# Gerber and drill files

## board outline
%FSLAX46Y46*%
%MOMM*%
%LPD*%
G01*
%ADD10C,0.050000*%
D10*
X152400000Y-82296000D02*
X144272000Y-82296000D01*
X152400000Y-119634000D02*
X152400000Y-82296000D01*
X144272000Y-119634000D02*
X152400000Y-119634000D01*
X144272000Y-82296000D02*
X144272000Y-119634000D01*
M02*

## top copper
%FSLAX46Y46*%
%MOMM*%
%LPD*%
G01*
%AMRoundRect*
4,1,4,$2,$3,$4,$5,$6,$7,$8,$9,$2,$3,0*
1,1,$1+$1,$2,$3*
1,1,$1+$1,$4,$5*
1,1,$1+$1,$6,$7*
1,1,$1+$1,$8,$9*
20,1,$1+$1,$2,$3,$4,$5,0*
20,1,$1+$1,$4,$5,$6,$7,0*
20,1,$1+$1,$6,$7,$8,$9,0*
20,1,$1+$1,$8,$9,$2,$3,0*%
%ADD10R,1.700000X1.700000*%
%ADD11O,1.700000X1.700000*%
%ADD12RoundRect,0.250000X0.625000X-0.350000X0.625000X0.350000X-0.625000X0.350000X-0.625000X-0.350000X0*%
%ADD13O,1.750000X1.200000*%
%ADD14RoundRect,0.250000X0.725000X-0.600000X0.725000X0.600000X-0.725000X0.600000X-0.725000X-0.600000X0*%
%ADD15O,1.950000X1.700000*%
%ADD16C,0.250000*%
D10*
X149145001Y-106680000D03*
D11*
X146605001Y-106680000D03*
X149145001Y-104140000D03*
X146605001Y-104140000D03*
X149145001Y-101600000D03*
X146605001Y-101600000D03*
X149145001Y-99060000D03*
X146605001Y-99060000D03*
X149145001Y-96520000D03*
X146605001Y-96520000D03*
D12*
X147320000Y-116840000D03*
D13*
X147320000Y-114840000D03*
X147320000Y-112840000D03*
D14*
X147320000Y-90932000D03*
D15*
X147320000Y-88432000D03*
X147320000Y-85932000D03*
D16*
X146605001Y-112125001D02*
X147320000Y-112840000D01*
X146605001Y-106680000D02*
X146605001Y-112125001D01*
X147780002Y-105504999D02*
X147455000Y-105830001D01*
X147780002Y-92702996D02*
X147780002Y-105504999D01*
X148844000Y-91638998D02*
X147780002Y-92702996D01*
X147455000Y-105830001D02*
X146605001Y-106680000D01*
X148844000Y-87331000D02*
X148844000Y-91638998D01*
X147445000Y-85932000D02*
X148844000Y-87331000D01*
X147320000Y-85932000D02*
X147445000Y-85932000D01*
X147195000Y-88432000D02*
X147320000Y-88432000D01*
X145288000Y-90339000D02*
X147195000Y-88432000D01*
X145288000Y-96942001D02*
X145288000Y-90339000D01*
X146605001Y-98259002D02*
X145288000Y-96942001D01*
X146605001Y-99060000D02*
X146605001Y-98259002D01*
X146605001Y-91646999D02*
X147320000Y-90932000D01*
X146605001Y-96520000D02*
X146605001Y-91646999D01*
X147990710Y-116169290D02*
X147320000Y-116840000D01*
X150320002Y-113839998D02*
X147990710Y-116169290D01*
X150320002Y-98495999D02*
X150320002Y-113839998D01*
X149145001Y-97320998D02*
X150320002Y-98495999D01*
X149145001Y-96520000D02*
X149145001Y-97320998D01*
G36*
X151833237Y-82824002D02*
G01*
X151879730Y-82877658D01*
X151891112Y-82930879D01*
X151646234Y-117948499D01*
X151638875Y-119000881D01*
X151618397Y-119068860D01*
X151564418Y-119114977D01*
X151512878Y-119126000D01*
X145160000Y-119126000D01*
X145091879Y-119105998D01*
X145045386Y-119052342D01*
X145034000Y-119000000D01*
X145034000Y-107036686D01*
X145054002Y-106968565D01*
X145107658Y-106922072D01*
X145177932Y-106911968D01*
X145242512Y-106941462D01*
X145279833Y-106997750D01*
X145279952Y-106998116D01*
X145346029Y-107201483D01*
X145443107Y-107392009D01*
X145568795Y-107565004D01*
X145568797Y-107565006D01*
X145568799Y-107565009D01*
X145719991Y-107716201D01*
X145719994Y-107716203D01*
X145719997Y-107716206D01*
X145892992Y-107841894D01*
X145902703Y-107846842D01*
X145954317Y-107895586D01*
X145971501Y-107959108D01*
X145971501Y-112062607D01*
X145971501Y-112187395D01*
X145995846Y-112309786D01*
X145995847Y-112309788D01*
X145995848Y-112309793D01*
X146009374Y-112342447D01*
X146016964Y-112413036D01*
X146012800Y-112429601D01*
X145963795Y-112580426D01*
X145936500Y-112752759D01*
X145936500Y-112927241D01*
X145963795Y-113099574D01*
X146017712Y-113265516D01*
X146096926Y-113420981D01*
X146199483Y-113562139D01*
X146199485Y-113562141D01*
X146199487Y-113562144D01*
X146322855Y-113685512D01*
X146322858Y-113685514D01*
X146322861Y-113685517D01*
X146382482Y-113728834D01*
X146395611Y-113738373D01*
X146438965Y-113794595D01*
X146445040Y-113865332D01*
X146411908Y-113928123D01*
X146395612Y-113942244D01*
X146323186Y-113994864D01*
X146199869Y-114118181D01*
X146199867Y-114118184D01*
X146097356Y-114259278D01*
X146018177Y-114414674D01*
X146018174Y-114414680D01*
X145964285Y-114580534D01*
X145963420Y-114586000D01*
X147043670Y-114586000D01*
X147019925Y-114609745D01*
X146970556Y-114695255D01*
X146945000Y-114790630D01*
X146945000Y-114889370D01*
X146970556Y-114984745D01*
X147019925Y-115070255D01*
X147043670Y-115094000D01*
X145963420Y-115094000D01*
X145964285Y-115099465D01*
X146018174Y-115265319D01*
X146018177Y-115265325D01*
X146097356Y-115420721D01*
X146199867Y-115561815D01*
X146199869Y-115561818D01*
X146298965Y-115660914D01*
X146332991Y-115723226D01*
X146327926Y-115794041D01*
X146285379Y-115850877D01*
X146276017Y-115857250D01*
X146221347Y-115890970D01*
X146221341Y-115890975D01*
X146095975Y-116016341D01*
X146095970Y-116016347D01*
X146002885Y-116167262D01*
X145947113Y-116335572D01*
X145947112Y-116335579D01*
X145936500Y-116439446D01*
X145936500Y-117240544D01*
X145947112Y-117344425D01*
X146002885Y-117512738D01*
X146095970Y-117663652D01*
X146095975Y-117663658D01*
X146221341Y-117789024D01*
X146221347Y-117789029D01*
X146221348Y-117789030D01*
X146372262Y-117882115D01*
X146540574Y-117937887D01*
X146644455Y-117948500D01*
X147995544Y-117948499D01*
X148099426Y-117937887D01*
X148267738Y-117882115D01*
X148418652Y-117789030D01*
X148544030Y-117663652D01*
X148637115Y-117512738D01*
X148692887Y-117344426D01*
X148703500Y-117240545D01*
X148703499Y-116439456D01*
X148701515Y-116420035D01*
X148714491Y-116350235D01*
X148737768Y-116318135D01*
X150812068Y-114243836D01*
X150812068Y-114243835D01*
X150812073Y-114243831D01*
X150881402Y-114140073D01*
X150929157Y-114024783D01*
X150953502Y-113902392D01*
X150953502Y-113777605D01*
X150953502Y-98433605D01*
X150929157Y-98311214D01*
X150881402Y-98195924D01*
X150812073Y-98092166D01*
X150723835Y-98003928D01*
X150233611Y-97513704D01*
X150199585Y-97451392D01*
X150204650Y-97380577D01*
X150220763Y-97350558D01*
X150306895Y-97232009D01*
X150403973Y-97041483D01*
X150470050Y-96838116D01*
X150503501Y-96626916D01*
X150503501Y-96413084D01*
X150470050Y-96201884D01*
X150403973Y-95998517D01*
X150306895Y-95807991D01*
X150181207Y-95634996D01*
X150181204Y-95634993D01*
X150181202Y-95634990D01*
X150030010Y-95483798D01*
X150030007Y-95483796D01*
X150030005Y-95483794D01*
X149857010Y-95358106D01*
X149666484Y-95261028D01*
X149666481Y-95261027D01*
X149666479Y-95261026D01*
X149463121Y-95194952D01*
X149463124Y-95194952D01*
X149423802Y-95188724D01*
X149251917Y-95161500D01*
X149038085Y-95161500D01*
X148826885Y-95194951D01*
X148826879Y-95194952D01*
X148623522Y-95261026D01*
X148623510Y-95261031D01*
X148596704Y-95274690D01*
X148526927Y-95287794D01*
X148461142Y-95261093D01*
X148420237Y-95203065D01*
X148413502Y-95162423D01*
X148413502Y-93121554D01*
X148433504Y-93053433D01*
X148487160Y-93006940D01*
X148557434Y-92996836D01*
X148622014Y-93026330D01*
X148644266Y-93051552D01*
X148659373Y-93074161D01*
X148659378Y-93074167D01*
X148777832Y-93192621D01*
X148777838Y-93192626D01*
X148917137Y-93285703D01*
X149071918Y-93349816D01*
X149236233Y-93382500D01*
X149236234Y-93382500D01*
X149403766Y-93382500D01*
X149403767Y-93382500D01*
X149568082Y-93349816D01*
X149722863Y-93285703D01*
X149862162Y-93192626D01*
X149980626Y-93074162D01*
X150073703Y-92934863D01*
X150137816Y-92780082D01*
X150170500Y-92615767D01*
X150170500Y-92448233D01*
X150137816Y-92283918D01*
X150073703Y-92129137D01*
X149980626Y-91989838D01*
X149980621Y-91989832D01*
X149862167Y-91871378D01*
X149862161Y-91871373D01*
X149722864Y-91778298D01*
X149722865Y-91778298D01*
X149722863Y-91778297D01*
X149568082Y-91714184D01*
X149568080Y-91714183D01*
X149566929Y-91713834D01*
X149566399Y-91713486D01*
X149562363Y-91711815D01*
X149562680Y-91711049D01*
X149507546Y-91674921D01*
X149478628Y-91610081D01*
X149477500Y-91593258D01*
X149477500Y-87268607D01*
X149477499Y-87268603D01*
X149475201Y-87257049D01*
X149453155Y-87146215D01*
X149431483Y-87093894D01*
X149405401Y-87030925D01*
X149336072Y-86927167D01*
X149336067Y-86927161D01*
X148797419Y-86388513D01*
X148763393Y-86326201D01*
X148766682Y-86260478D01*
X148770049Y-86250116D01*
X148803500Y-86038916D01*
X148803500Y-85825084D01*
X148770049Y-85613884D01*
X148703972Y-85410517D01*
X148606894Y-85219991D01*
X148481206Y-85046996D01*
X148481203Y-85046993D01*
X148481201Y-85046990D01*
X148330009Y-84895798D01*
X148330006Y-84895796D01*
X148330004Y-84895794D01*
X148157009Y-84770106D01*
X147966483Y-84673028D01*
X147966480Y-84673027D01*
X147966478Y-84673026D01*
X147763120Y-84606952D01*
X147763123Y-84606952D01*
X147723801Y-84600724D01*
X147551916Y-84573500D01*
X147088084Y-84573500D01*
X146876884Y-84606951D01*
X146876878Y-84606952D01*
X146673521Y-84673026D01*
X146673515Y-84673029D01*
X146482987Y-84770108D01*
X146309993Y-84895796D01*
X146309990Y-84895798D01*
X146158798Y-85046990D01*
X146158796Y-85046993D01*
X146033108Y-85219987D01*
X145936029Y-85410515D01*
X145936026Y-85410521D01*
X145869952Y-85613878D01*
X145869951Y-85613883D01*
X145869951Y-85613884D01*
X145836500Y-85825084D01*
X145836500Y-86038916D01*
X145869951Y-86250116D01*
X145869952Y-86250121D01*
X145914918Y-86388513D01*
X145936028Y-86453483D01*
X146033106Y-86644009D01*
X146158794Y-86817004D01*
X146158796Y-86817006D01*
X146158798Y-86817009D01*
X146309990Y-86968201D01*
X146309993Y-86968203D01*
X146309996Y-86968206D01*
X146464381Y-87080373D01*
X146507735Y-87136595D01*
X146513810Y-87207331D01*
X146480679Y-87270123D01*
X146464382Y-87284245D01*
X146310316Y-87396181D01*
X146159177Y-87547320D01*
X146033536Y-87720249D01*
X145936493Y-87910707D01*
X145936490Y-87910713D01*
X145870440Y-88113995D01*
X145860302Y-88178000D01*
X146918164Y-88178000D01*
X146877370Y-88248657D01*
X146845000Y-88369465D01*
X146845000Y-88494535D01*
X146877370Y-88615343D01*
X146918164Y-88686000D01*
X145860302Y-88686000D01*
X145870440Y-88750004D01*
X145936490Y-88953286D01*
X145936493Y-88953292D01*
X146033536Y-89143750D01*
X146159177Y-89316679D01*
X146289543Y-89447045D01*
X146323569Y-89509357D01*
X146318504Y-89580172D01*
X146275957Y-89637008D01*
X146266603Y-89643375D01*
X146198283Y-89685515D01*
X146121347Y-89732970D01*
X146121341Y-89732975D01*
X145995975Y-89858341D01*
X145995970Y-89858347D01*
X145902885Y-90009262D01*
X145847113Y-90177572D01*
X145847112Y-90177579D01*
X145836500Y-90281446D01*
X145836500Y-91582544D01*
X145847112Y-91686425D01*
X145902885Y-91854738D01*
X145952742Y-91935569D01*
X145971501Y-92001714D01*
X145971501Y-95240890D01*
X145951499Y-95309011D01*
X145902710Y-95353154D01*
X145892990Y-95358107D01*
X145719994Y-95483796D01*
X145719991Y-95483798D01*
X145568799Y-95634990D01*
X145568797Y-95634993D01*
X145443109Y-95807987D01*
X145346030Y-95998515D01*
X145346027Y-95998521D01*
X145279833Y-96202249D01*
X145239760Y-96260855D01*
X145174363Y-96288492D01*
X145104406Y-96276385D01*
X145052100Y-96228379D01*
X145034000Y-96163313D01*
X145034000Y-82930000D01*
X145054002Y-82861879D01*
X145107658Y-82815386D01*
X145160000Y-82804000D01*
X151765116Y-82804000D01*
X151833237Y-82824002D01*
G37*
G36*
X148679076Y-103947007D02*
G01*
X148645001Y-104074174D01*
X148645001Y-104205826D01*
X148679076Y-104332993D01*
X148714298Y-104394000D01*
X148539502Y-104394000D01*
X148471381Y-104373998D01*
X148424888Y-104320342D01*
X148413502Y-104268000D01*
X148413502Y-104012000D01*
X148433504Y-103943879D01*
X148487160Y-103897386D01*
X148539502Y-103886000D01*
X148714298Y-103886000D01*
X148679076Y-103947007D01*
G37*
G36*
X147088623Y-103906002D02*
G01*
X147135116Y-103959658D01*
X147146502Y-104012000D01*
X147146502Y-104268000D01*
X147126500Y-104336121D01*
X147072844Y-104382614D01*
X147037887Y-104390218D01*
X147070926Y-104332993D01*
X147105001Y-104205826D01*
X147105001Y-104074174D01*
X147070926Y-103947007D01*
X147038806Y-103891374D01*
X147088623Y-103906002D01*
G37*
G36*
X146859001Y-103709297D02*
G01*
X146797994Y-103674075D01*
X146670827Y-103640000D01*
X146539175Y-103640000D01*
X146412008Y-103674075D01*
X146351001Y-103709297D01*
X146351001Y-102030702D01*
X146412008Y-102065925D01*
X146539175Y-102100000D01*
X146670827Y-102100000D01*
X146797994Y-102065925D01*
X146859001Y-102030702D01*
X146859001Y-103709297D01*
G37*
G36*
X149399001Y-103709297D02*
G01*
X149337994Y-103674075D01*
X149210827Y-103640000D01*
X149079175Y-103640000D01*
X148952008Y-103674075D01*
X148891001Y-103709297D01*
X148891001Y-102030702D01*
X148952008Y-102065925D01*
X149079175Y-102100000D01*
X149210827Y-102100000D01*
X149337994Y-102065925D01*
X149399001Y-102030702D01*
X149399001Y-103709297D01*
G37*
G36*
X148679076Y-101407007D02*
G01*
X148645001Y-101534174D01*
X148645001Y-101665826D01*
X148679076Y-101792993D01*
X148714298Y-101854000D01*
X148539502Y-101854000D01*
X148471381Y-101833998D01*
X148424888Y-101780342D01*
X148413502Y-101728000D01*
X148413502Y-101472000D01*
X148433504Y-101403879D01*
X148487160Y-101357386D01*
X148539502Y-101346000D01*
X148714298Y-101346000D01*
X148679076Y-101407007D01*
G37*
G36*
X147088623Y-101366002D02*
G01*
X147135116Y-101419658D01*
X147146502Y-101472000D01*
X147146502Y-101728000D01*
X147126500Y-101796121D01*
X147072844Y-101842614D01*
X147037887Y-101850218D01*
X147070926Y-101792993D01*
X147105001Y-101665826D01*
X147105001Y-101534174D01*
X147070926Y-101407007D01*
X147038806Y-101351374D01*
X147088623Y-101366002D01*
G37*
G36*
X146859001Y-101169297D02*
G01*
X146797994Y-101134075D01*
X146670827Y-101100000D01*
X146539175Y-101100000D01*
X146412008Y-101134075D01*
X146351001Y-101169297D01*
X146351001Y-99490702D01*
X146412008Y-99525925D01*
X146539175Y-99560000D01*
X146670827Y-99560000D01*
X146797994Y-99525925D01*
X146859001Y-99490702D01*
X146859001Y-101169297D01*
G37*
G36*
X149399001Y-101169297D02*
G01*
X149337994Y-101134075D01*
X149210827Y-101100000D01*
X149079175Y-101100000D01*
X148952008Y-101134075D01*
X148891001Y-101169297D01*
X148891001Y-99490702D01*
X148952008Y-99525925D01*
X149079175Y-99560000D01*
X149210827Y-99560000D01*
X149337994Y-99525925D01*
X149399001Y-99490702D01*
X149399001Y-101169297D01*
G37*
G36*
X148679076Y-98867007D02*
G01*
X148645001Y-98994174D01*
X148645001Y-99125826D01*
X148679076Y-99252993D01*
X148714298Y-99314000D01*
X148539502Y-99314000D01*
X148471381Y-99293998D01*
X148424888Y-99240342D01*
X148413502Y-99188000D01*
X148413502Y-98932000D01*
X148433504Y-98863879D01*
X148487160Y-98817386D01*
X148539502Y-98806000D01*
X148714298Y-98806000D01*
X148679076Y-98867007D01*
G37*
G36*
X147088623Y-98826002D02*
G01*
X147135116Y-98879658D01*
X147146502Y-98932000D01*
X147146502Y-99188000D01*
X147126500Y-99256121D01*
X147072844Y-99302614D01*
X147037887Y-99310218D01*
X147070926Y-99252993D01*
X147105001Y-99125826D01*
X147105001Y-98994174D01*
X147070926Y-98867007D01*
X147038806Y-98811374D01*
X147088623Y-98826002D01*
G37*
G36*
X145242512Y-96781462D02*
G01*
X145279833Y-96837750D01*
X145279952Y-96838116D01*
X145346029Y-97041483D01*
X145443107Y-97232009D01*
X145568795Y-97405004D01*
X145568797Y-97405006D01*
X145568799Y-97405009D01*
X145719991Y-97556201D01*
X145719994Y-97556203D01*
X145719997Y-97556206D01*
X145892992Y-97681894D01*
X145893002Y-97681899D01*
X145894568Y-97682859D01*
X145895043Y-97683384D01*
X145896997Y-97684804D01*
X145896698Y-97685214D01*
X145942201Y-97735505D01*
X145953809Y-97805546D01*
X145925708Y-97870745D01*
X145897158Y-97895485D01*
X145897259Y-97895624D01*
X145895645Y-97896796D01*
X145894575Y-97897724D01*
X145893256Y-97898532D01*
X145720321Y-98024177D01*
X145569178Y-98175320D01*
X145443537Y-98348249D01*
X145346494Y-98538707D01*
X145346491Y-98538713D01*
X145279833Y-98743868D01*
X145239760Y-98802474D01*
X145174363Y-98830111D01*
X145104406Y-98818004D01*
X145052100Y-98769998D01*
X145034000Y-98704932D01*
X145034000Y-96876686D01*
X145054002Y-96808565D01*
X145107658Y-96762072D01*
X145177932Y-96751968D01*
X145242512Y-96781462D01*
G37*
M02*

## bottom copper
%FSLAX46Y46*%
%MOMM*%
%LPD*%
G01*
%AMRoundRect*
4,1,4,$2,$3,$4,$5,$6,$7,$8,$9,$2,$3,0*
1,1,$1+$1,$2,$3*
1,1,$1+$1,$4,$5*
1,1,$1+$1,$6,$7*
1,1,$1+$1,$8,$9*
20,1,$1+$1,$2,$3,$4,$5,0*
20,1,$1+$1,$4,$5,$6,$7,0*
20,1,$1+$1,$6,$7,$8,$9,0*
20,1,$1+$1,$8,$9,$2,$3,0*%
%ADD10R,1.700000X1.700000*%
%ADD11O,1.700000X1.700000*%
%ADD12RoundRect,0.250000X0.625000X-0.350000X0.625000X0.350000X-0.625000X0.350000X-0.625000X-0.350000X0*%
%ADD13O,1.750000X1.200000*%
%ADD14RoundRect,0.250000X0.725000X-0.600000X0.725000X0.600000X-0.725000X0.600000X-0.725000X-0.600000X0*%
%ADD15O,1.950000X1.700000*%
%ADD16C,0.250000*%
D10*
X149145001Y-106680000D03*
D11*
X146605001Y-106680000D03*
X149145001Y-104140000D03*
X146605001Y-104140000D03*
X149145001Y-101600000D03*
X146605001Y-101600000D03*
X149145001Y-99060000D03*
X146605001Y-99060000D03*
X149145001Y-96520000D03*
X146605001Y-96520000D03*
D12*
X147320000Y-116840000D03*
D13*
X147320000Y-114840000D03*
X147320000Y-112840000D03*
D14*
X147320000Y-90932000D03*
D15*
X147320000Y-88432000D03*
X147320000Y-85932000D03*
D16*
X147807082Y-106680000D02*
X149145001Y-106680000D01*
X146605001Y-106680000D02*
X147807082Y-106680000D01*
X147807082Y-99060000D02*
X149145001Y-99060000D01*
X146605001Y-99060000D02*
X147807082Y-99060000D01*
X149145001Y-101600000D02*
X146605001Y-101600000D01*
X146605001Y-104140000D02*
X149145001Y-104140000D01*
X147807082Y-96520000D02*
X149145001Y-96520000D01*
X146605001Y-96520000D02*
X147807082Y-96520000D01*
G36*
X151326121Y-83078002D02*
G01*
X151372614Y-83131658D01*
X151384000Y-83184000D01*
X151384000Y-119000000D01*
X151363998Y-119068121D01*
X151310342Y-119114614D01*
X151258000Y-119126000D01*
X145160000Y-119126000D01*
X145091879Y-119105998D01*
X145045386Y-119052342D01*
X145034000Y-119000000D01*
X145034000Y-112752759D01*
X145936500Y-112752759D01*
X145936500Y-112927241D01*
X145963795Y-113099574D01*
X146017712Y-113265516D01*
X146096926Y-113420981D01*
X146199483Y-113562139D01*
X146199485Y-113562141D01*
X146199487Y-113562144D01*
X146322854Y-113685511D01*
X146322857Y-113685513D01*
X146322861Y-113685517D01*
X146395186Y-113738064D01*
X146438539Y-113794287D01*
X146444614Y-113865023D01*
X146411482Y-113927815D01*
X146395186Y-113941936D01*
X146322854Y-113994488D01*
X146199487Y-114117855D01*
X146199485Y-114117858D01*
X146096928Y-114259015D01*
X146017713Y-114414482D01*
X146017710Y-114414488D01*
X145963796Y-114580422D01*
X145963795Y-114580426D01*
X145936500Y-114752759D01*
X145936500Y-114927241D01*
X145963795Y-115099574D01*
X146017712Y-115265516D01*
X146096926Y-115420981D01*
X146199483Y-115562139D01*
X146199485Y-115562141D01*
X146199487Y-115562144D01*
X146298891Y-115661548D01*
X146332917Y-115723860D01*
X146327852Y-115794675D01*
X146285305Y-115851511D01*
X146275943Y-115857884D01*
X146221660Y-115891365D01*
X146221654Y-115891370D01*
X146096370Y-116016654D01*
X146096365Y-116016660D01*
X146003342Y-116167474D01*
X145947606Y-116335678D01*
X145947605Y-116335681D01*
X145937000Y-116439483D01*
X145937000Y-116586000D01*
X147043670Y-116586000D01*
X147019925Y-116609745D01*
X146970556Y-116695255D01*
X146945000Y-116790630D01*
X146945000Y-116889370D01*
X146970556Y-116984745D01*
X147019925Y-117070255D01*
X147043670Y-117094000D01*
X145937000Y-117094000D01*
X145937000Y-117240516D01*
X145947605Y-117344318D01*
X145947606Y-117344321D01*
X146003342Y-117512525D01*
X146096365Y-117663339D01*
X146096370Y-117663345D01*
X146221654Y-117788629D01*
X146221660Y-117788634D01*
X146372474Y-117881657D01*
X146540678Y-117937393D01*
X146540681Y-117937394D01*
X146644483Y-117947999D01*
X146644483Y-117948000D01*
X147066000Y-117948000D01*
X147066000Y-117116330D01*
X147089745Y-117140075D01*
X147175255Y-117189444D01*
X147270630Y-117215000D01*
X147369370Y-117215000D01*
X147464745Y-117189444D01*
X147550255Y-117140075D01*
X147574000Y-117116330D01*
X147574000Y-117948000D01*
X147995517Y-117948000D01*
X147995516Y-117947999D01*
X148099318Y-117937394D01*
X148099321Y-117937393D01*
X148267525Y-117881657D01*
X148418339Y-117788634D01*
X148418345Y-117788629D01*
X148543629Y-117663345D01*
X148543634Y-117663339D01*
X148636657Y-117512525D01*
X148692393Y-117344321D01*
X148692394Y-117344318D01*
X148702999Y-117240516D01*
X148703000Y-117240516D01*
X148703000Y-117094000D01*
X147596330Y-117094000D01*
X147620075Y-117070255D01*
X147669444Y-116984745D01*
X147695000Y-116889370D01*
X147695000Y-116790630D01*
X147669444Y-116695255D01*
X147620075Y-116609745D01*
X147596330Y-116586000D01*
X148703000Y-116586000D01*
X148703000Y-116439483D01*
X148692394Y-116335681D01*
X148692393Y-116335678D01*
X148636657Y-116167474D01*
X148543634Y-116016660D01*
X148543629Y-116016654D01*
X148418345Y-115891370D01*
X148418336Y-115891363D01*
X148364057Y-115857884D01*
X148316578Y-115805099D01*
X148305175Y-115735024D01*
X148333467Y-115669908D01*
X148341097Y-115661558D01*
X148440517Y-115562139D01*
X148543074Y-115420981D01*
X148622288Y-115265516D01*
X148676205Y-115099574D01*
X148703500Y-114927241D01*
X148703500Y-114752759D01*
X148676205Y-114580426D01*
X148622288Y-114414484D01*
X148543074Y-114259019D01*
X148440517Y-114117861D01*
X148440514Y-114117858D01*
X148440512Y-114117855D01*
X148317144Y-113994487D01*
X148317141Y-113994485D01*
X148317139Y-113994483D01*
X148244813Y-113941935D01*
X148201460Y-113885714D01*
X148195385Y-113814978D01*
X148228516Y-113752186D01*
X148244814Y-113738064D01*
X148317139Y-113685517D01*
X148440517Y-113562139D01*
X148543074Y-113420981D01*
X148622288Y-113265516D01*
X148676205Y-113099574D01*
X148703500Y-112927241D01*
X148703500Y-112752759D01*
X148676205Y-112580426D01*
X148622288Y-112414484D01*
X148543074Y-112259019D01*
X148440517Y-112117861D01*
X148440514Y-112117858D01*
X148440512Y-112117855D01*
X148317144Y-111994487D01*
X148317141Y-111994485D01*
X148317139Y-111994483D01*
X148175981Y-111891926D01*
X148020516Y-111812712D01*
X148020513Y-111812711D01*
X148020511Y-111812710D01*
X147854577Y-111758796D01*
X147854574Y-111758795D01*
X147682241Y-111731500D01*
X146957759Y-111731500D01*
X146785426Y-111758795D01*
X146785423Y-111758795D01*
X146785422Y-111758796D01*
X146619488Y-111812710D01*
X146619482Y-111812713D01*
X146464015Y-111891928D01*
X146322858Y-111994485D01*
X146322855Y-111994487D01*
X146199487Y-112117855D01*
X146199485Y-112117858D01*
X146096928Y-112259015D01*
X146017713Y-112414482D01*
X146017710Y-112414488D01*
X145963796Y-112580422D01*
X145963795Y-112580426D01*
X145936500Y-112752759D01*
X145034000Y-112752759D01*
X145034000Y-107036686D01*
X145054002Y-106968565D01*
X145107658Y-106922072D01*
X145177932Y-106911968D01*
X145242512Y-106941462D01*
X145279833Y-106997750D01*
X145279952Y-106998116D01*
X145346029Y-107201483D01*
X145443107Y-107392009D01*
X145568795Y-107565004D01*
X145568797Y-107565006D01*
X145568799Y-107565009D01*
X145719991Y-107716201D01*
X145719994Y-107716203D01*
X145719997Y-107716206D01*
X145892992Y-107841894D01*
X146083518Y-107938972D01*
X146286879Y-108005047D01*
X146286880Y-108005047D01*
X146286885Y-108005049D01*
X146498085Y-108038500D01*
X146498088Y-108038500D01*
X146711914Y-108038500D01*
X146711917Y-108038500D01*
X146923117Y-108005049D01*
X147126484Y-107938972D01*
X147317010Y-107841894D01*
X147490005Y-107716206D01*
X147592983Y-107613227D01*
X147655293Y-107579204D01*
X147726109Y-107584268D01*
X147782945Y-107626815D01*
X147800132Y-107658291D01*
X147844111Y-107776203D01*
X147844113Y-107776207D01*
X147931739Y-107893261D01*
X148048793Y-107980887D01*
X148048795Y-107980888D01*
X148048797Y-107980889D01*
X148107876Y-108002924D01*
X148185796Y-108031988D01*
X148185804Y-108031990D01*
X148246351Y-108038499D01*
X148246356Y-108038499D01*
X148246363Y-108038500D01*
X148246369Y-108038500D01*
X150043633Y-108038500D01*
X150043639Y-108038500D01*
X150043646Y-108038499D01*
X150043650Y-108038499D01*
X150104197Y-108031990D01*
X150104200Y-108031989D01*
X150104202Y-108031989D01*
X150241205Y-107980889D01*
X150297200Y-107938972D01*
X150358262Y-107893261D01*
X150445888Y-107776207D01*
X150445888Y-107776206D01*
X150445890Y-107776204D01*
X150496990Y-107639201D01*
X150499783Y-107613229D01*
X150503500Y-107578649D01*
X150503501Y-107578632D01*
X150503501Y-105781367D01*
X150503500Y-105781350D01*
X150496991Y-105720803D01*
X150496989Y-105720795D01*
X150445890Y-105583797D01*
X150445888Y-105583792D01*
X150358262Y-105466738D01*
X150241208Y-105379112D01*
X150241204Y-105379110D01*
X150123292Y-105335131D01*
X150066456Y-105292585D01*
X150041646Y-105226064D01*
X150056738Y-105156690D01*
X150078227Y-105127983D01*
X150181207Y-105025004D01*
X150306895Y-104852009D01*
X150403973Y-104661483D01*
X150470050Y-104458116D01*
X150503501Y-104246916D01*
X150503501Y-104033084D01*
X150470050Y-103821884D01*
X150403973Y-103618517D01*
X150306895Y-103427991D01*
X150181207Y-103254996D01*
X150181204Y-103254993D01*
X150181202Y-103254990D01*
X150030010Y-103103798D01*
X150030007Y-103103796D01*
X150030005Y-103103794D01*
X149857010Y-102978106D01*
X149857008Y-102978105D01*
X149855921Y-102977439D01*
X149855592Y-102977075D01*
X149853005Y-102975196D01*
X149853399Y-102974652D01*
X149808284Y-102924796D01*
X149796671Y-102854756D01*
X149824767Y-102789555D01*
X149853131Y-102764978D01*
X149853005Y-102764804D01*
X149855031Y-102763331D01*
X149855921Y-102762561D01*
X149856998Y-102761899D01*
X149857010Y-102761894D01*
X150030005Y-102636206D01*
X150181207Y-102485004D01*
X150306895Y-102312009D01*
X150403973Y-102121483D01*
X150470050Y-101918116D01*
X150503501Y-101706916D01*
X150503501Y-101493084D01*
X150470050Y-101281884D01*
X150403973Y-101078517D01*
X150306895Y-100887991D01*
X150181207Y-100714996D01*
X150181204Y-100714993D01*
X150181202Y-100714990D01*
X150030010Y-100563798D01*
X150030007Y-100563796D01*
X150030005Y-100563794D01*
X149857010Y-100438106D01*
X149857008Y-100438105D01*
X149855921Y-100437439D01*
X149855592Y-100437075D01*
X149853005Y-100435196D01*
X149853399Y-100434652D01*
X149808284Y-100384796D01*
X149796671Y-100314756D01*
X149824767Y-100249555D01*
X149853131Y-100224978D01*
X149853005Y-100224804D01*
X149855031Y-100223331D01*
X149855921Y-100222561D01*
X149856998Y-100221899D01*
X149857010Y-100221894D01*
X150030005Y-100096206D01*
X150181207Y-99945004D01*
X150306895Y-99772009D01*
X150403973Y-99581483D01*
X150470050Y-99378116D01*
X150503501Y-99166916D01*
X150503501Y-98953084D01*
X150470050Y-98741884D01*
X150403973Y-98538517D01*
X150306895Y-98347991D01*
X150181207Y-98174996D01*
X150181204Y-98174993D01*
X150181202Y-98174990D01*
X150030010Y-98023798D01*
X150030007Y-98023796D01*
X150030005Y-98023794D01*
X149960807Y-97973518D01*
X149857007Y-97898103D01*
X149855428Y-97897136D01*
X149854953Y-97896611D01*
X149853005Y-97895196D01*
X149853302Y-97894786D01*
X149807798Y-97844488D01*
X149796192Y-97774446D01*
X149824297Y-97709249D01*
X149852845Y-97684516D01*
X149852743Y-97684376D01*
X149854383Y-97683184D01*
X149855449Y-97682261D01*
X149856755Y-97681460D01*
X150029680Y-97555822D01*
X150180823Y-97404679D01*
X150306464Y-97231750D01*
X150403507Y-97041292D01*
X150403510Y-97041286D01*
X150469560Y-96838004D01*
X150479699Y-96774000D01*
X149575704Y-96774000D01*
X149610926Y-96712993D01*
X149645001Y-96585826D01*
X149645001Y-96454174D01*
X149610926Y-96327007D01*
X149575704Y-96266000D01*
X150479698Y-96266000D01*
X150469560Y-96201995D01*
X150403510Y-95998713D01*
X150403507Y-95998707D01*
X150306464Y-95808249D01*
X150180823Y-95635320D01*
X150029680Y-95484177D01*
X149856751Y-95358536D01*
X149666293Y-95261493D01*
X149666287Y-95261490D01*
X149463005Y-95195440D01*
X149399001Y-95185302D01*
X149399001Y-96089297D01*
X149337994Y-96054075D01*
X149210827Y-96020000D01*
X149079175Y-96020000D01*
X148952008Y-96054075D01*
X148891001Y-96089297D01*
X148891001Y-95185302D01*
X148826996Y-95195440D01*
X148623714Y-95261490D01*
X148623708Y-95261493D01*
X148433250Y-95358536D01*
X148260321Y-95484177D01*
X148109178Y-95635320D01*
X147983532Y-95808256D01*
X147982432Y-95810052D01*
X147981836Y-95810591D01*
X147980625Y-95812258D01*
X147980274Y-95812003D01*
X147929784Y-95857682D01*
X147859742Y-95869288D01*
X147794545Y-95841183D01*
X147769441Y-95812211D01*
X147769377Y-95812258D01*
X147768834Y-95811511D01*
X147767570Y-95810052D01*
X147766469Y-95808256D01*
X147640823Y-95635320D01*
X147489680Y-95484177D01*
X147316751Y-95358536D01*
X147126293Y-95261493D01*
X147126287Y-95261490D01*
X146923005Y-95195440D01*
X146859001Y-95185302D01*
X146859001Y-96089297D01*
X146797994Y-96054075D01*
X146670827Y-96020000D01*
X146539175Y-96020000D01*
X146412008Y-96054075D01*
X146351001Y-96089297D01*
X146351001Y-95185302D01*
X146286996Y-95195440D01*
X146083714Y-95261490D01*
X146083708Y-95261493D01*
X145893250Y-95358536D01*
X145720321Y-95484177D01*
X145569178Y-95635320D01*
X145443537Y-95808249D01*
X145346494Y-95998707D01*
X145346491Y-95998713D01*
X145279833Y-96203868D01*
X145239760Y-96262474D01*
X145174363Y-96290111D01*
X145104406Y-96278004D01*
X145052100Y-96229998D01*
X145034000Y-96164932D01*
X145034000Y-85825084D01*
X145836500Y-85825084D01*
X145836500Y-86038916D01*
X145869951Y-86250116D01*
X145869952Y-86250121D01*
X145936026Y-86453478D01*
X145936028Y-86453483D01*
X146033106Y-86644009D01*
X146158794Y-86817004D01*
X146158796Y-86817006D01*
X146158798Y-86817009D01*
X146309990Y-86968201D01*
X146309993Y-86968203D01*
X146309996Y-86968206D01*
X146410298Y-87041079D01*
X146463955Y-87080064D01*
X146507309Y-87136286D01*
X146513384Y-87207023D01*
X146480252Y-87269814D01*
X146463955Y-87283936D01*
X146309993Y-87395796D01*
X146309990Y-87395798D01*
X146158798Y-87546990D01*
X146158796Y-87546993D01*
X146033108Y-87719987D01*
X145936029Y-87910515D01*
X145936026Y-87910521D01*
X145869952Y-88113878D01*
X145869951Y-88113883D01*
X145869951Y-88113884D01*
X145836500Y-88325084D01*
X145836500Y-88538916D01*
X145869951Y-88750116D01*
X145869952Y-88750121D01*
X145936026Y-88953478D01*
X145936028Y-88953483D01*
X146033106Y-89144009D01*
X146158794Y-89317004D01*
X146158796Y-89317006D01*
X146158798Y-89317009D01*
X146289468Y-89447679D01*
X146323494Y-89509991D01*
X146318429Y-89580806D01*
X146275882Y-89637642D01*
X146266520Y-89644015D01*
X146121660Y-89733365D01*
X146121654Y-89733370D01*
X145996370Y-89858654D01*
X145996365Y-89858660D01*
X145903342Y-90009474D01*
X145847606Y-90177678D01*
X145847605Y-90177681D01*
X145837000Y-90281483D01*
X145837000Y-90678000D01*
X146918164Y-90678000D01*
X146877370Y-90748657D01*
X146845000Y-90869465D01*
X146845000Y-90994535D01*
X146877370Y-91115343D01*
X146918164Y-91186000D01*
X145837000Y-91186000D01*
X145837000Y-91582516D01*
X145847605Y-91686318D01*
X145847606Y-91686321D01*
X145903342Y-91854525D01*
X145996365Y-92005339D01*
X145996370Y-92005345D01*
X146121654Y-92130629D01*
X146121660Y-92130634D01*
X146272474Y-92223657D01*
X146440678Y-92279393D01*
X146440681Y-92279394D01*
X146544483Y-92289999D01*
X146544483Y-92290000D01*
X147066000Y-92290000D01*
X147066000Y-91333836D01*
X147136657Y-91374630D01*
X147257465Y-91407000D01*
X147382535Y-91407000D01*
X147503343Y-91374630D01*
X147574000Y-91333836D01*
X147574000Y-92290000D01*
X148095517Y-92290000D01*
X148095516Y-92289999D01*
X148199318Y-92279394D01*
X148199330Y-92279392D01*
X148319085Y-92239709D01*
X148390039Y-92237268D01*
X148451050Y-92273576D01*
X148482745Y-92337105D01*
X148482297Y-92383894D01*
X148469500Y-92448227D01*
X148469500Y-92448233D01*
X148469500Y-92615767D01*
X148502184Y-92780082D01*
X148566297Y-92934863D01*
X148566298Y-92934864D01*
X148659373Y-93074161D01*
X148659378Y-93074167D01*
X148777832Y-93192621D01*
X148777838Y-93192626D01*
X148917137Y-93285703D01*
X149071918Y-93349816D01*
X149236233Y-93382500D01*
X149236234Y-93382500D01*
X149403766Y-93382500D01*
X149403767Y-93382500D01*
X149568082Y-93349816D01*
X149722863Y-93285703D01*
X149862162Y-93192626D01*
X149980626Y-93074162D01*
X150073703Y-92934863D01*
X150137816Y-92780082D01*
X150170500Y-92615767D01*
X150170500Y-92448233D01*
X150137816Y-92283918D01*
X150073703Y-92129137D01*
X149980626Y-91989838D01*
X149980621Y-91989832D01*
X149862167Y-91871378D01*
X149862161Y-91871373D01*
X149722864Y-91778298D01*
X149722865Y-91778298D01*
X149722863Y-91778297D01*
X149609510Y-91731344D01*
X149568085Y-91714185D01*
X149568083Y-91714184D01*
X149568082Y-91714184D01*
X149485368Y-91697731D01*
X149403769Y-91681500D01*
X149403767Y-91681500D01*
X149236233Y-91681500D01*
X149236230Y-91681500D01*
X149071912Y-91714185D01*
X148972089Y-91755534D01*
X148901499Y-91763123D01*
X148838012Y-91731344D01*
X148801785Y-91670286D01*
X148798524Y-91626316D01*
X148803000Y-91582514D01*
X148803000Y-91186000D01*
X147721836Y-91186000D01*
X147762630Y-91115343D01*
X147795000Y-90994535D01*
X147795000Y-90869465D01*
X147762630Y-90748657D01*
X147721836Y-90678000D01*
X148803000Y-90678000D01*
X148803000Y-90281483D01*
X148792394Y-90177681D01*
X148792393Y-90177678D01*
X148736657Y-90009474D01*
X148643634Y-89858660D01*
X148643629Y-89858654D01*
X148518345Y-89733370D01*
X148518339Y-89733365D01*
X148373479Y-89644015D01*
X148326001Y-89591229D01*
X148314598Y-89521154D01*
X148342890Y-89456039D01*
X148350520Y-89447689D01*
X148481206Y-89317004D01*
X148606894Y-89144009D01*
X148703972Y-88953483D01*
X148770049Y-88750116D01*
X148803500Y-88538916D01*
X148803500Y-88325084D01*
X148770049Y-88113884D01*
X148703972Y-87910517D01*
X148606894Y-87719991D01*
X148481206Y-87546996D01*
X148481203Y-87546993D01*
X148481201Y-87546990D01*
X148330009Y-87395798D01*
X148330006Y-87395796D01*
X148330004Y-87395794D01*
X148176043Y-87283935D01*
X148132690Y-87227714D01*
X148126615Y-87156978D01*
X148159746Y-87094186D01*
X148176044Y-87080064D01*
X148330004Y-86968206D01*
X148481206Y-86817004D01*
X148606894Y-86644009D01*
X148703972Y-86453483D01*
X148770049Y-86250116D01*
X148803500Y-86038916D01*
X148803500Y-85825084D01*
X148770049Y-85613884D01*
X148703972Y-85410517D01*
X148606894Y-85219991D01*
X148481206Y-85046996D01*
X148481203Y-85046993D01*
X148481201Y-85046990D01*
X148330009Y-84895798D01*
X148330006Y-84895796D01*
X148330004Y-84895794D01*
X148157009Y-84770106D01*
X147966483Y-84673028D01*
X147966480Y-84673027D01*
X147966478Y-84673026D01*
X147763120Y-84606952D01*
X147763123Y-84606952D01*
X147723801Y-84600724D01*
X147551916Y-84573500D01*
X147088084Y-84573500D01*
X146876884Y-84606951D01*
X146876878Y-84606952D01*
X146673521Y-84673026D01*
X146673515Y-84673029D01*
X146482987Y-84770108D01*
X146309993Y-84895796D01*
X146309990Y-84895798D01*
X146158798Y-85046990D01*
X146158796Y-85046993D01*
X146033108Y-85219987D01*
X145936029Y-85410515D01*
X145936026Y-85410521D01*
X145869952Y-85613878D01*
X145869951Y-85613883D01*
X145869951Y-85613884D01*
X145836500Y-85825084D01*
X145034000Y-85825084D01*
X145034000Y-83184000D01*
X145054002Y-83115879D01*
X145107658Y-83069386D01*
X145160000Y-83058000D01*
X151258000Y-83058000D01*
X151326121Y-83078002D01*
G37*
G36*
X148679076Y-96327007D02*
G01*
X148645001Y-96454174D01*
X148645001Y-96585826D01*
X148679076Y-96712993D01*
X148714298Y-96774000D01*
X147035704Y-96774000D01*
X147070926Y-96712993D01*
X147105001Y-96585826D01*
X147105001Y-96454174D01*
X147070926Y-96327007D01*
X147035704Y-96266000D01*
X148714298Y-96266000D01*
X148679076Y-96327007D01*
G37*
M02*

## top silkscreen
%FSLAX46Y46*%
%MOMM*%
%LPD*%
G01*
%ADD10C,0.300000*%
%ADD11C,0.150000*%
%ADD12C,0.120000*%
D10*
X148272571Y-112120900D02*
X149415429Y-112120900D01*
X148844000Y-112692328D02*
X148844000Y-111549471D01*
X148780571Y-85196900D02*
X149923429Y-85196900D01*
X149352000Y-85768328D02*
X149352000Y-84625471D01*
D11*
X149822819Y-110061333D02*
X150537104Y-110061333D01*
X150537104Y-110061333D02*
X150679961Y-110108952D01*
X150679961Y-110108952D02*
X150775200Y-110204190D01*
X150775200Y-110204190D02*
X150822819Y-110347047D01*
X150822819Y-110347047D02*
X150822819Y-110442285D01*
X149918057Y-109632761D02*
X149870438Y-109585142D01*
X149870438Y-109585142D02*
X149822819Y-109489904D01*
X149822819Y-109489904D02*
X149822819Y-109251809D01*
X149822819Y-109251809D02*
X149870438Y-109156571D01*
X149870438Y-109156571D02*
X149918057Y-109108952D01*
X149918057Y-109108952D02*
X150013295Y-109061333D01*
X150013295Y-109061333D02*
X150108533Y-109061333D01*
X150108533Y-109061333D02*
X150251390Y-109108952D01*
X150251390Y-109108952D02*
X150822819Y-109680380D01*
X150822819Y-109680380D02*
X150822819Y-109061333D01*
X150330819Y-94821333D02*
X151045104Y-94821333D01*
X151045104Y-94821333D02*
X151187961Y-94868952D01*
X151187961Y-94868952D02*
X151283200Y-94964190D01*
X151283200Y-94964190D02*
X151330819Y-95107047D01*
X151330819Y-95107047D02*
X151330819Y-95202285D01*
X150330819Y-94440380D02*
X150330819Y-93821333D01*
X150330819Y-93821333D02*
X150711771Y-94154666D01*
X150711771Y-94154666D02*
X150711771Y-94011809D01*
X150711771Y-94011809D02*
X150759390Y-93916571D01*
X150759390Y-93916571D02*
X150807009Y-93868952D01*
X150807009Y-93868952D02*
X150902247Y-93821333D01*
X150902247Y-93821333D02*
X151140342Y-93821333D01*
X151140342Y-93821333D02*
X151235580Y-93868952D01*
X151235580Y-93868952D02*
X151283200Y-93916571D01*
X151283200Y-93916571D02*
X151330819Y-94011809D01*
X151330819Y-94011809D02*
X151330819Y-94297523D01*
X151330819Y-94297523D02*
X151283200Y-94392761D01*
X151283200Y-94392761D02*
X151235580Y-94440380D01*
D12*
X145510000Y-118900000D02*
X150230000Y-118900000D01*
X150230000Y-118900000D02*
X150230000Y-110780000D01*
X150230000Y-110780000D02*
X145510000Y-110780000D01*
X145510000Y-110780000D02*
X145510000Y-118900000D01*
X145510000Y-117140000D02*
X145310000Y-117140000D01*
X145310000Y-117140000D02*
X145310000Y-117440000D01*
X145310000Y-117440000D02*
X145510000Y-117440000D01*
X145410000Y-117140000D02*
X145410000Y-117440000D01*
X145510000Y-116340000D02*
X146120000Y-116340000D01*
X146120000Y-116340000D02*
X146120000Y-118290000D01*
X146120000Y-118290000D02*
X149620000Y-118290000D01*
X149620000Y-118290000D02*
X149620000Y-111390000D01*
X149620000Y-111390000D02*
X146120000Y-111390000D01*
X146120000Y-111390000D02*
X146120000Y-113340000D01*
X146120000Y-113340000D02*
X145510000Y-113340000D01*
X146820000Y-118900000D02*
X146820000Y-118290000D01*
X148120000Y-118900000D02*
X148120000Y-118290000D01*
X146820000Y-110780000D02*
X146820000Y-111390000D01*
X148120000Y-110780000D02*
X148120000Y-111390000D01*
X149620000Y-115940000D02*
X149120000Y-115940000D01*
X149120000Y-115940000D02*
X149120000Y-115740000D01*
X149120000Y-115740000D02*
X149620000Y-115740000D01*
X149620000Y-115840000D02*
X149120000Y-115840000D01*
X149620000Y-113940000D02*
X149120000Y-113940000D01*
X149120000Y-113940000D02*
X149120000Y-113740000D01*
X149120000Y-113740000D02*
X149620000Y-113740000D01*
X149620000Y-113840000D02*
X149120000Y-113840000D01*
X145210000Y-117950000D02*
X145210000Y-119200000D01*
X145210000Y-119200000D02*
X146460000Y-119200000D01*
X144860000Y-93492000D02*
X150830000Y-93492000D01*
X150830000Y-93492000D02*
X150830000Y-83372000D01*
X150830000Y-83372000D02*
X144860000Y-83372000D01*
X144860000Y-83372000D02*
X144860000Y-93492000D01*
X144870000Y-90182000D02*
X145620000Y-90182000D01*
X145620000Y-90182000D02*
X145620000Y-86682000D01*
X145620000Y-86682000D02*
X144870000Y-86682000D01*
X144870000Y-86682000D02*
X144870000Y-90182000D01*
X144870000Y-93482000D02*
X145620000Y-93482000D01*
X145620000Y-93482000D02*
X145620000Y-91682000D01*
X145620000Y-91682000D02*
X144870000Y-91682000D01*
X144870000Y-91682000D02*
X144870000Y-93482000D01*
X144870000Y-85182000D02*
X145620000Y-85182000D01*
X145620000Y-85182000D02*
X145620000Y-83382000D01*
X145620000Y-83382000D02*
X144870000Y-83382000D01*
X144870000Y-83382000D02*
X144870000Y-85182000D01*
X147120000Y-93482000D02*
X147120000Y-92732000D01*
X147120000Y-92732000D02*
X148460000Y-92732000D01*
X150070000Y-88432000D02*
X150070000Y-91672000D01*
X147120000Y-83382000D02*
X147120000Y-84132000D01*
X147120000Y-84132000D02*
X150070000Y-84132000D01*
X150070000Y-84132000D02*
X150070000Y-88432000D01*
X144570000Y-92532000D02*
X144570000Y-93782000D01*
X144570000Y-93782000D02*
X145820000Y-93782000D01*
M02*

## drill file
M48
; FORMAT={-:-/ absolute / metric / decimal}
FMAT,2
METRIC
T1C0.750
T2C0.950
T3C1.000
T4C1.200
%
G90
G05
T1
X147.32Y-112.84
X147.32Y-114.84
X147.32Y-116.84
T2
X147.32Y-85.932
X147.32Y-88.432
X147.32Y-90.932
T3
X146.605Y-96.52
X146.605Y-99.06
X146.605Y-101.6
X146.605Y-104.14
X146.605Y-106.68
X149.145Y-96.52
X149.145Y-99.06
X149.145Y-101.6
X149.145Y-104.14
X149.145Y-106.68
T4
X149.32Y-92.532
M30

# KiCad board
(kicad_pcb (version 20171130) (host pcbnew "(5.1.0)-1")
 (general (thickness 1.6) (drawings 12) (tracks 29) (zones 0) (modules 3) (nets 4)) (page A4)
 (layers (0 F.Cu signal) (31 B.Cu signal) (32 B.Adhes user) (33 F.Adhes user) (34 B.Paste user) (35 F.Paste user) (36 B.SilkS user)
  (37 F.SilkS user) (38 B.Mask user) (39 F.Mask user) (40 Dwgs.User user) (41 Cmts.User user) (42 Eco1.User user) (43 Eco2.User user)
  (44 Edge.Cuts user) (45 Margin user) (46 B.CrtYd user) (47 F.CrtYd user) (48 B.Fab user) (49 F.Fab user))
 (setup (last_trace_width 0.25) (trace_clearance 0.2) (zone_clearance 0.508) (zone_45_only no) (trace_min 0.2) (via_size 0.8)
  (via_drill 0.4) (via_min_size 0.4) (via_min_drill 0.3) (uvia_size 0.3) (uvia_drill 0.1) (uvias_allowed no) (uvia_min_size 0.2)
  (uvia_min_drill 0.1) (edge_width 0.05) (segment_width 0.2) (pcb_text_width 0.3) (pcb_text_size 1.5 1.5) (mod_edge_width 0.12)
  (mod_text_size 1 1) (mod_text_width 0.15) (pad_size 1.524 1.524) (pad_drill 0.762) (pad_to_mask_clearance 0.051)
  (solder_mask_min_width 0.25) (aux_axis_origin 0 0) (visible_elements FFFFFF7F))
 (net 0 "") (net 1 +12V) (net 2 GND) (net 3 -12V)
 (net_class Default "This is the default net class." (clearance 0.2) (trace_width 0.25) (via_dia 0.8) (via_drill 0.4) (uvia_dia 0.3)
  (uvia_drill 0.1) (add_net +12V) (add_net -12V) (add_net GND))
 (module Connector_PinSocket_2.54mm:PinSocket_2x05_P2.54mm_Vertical (layer B.Cu) (at 149.145001 106.68)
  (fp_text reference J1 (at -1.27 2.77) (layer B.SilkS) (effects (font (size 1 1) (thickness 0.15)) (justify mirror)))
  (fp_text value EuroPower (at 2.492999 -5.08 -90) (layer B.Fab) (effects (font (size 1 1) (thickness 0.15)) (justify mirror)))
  (pad 1 thru_hole rect (at 0 0) (size 1.7 1.7) (drill 1) (layers *.Cu *.Mask) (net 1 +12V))
  (pad 2 thru_hole oval (at -2.54 0) (size 1.7 1.7) (drill 1) (layers *.Cu *.Mask) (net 1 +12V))
  (pad 3 thru_hole oval (at 0 -2.54) (size 1.7 1.7) (drill 1) (layers *.Cu *.Mask) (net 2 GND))
  (pad 4 thru_hole oval (at -2.54 -2.54) (size 1.7 1.7) (drill 1) (layers *.Cu *.Mask) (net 2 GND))
  (pad 5 thru_hole oval (at 0 -5.08) (size 1.7 1.7) (drill 1) (layers *.Cu *.Mask) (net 2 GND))
  (pad 6 thru_hole oval (at -2.54 -5.08) (size 1.7 1.7) (drill 1) (layers *.Cu *.Mask) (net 2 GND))
  (pad 7 thru_hole oval (at 0 -7.62) (size 1.7 1.7) (drill 1) (layers *.Cu *.Mask) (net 2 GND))
  (pad 8 thru_hole oval (at -2.54 -7.62) (size 1.7 1.7) (drill 1) (layers *.Cu *.Mask) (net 2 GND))
  (pad 9 thru_hole oval (at 0 -10.16) (size 1.7 1.7) (drill 1) (layers *.Cu *.Mask) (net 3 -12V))
  (pad 10 thru_hole oval (at -2.54 -10.16) (size 1.7 1.7) (drill 1) (layers *.Cu *.Mask) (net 3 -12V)))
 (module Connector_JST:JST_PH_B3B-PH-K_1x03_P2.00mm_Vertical (layer F.Cu) (at 147.32 116.84 90)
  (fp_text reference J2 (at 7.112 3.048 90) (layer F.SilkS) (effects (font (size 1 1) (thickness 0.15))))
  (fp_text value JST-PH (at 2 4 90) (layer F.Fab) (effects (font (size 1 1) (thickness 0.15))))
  (fp_line (start -2.06 -1.81) (end -2.06 2.91) (layer F.SilkS) (width 0.12))
  (fp_line (start -2.06 2.91) (end 6.06 2.91) (layer F.SilkS) (width 0.12))
  (fp_line (start 6.06 2.91) (end 6.06 -1.81) (layer F.SilkS) (width 0.12))
  (fp_line (start 6.06 -1.81) (end -2.06 -1.81) (layer F.SilkS) (width 0.12))
  (fp_line (start -0.3 -1.81) (end -0.3 -2.01) (layer F.SilkS) (width 0.12))
  (fp_line (start -0.3 -2.01) (end -0.6 -2.01) (layer F.SilkS) (width 0.12))
  (fp_line (start -0.6 -2.01) (end -0.6 -1.81) (layer F.SilkS) (width 0.12))
  (fp_line (start -0.3 -1.91) (end -0.6 -1.91) (layer F.SilkS) (width 0.12))
  (fp_line (start 0.5 -1.81) (end 0.5 -1.2) (layer F.SilkS) (width 0.12))
  (fp_line (start 0.5 -1.2) (end -1.45 -1.2) (layer F.SilkS) (width 0.12))
  (fp_line (start -1.45 -1.2) (end -1.45 2.3) (layer F.SilkS) (width 0.12))
  (fp_line (start -1.45 2.3) (end 5.45 2.3) (layer F.SilkS) (width 0.12))
  (fp_line (start 5.45 2.3) (end 5.45 -1.2) (layer F.SilkS) (width 0.12))
  (fp_line (start 5.45 -1.2) (end 3.5 -1.2) (layer F.SilkS) (width 0.12))
  (fp_line (start 3.5 -1.2) (end 3.5 -1.81) (layer F.SilkS) (width 0.12))
  (fp_line (start -2.06 -0.5) (end -1.45 -0.5) (layer F.SilkS) (width 0.12))
  (fp_line (start -2.06 0.8) (end -1.45 0.8) (layer F.SilkS) (width 0.12))
  (fp_line (start 6.06 -0.5) (end 5.45 -0.5) (layer F.SilkS) (width 0.12))
  (fp_line (start 6.06 0.8) (end 5.45 0.8) (layer F.SilkS) (width 0.12))
  (fp_line (start 0.9 2.3) (end 0.9 1.8) (layer F.SilkS) (width 0.12))
  (fp_line (start 0.9 1.8) (end 1.1 1.8) (layer F.SilkS) (width 0.12))
  (fp_line (start 1.1 1.8) (end 1.1 2.3) (layer F.SilkS) (width 0.12))
  (fp_line (start 1 2.3) (end 1 1.8) (layer F.SilkS) (width 0.12))
  (fp_line (start 2.9 2.3) (end 2.9 1.8) (layer F.SilkS) (width 0.12))
  (fp_line (start 2.9 1.8) (end 3.1 1.8) (layer F.SilkS) (width 0.12))
  (fp_line (start 3.1 1.8) (end 3.1 2.3) (layer F.SilkS) (width 0.12))
  (fp_line (start 3 2.3) (end 3 1.8) (layer F.SilkS) (width 0.12))
  (fp_line (start -1.11 -2.11) (end -2.36 -2.11) (layer F.SilkS) (width 0.12))
  (fp_line (start -2.36 -2.11) (end -2.36 -0.86) (layer F.SilkS) (width 0.12))
  (pad 1 thru_hole roundrect (at 0 0 90) (size 1.2 1.75) (drill 0.75) (layers *.Cu *.Mask) (roundrect_rratio 0.208333) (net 3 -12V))
  (pad 2 thru_hole oval (at 2 0 90) (size 1.2 1.75) (drill 0.75) (layers *.Cu *.Mask) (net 2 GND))
  (pad 3 thru_hole oval (at 4 0 90) (size 1.2 1.75) (drill 0.75) (layers *.Cu *.Mask) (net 1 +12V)))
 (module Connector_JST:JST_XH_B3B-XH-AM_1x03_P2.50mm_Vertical (layer F.Cu) (at 147.32 90.932 90)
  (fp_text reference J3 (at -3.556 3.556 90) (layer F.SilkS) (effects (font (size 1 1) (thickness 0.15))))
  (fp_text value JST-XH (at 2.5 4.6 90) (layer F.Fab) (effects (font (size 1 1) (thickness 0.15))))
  (fp_line (start -2.56 -2.46) (end -2.56 3.51) (layer F.SilkS) (width 0.12))
  (fp_line (start -2.56 3.51) (end 7.56 3.51) (layer F.SilkS) (width 0.12))
  (fp_line (start 7.56 3.51) (end 7.56 -2.46) (layer F.SilkS) (width 0.12))
  (fp_line (start 7.56 -2.46) (end -2.56 -2.46) (layer F.SilkS) (width 0.12))
  (fp_line (start 0.75 -2.45) (end 0.75 -1.7) (layer F.SilkS) (width 0.12))
  (fp_line (start 0.75 -1.7) (end 4.25 -1.7) (layer F.SilkS) (width 0.12))
  (fp_line (start 4.25 -1.7) (end 4.25 -2.45) (layer F.SilkS) (width 0.12))
  (fp_line (start 4.25 -2.45) (end 0.75 -2.45) (layer F.SilkS) (width 0.12))
  (fp_line (start -2.55 -2.45) (end -2.55 -1.7) (layer F.SilkS) (width 0.12))
  (fp_line (start -2.55 -1.7) (end -0.75 -1.7) (layer F.SilkS) (width 0.12))
  (fp_line (start -0.75 -1.7) (end -0.75 -2.45) (layer F.SilkS) (width 0.12))
  (fp_line (start -0.75 -2.45) (end -2.55 -2.45) (layer F.SilkS) (width 0.12))
  (fp_line (start 5.75 -2.45) (end 5.75 -1.7) (layer F.SilkS) (width 0.12))
  (fp_line (start 5.75 -1.7) (end 7.55 -1.7) (layer F.SilkS) (width 0.12))
  (fp_line (start 7.55 -1.7) (end 7.55 -2.45) (layer F.SilkS) (width 0.12))
  (fp_line (start 7.55 -2.45) (end 5.75 -2.45) (layer F.SilkS) (width 0.12))
  (fp_line (start -2.55 -0.2) (end -1.8 -0.2) (layer F.SilkS) (width 0.12))
  (fp_line (start -1.8 -0.2) (end -1.8 1.14) (layer F.SilkS) (width 0.12))
  (fp_line (start 2.5 2.75) (end -0.74 2.75) (layer F.SilkS) (width 0.12))
  (fp_line (start 7.55 -0.2) (end 6.8 -0.2) (layer F.SilkS) (width 0.12))
  (fp_line (start 6.8 -0.2) (end 6.8 2.75) (layer F.SilkS) (width 0.12))
  (fp_line (start 6.8 2.75) (end 2.5 2.75) (layer F.SilkS) (width 0.12))
  (fp_line (start -1.6 -2.75) (end -2.85 -2.75) (layer F.SilkS) (width 0.12))
  (fp_line (start -2.85 -2.75) (end -2.85 -1.5) (layer F.SilkS) (width 0.12))
  (pad 1 thru_hole roundrect (at 0 0 90) (size 1.7 1.95) (drill 0.95) (layers *.Cu *.Mask) (roundrect_rratio 0.147059) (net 3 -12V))
  (pad 2 thru_hole oval (at 2.5 0 90) (size 1.7 1.95) (drill 0.95) (layers *.Cu *.Mask) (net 2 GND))
  (pad 3 thru_hole oval (at 5 0 90) (size 1.7 1.95) (drill 0.95) (layers *.Cu *.Mask) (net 1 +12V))
  (pad "" np_thru_hole circle (at -1.6 2 90) (size 1.2 1.2) (drill 1.2) (layers *.Cu *.Mask)))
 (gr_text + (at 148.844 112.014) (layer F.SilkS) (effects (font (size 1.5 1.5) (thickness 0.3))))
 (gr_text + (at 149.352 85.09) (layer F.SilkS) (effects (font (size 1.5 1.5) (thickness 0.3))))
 (gr_line (start 152.4 82.296) (end 144.272 82.296) (layer Edge.Cuts) (width 0.05))
 (gr_line (start 152.4 119.634) (end 152.4 82.296) (layer Edge.Cuts) (width 0.05))
 (gr_line (start 144.272 119.634) (end 152.4 119.634) (layer Edge.Cuts) (width 0.05))
 (gr_line (start 144.272 82.296) (end 144.272 119.634) (layer Edge.Cuts) (width 0.05))
 (segment (start 146.605001 112.125001) (end 147.32 112.84) (width 0.25) (layer F.Cu) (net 1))
 (segment (start 146.605001 106.68) (end 146.605001 112.125001) (width 0.25) (layer F.Cu) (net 1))
 (segment (start 147.780002 105.504999) (end 147.455 105.830001) (width 0.25) (layer F.Cu) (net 1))
 (segment (start 147.780002 92.702996) (end 147.780002 105.504999) (width 0.25) (layer F.Cu) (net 1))
 (segment (start 148.844 91.638998) (end 147.780002 92.702996) (width 0.25) (layer F.Cu) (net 1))
 (segment (start 147.455 105.830001) (end 146.605001 106.68) (width 0.25) (layer F.Cu) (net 1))
 (segment (start 148.844 87.331) (end 148.844 91.638998) (width 0.25) (layer F.Cu) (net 1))
 (segment (start 147.445 85.932) (end 148.844 87.331) (width 0.25) (layer F.Cu) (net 1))
 (segment (start 147.32 85.932) (end 147.445 85.932) (width 0.25) (layer F.Cu) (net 1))
 (segment (start 147.807082 106.68) (end 149.145001 106.68) (width 0.25) (layer B.Cu) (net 1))
 (segment (start 146.605001 106.68) (end 147.807082 106.68) (width 0.25) (layer B.Cu) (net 1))
 (segment (start 147.807082 99.06) (end 149.145001 99.06) (width 0.25) (layer B.Cu) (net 2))
 (segment (start 146.605001 99.06) (end 147.807082 99.06) (width 0.25) (layer B.Cu) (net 2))
 (segment (start 149.145001 101.6) (end 146.605001 101.6) (width 0.25) (layer B.Cu) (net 2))
 (segment (start 146.605001 104.14) (end 149.145001 104.14) (width 0.25) (layer B.Cu) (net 2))
 (segment (start 147.195 88.432) (end 147.32 88.432) (width 0.25) (layer F.Cu) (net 2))
 (segment (start 145.288 90.339) (end 147.195 88.432) (width 0.25) (layer F.Cu) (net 2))
 (segment (start 145.288 96.942001) (end 145.288 90.339) (width 0.25) (layer F.Cu) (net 2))
 (segment (start 146.605001 98.259002) (end 145.288 96.942001) (width 0.25) (layer F.Cu) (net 2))
 (segment (start 146.605001 99.06) (end 146.605001 98.259002) (width 0.25) (layer F.Cu) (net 2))
 (segment (start 146.605001 91.646999) (end 147.32 90.932) (width 0.25) (layer F.Cu) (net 3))
 (segment (start 146.605001 96.52) (end 146.605001 91.646999) (width 0.25) (layer F.Cu) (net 3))
 (segment (start 147.807082 96.52) (end 149.145001 96.52) (width 0.25) (layer B.Cu) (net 3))
 (segment (start 146.605001 96.52) (end 147.807082 96.52) (width 0.25) (layer B.Cu) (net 3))
 (segment (start 147.99071 116.16929) (end 147.32 116.84) (width 0.25) (layer F.Cu) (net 3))
 (segment (start 150.320002 113.839998) (end 147.99071 116.16929) (width 0.25) (layer F.Cu) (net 3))
 (segment (start 150.320002 98.495999) (end 150.320002 113.839998) (width 0.25) (layer F.Cu) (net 3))
 (segment (start 149.145001 97.320998) (end 150.320002 98.495999) (width 0.25) (layer F.Cu) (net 3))
 (segment (start 149.145001 96.52) (end 149.145001 97.320998) (width 0.25) (layer F.Cu) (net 3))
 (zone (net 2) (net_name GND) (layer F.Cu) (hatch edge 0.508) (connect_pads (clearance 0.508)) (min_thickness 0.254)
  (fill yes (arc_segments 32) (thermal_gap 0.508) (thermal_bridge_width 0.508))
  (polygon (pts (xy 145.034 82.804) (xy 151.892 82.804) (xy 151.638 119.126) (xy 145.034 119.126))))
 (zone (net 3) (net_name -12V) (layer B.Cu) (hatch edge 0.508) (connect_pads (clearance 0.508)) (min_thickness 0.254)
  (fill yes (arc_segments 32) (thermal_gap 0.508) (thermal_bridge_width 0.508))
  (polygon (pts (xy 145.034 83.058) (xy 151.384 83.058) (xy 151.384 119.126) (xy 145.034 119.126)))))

